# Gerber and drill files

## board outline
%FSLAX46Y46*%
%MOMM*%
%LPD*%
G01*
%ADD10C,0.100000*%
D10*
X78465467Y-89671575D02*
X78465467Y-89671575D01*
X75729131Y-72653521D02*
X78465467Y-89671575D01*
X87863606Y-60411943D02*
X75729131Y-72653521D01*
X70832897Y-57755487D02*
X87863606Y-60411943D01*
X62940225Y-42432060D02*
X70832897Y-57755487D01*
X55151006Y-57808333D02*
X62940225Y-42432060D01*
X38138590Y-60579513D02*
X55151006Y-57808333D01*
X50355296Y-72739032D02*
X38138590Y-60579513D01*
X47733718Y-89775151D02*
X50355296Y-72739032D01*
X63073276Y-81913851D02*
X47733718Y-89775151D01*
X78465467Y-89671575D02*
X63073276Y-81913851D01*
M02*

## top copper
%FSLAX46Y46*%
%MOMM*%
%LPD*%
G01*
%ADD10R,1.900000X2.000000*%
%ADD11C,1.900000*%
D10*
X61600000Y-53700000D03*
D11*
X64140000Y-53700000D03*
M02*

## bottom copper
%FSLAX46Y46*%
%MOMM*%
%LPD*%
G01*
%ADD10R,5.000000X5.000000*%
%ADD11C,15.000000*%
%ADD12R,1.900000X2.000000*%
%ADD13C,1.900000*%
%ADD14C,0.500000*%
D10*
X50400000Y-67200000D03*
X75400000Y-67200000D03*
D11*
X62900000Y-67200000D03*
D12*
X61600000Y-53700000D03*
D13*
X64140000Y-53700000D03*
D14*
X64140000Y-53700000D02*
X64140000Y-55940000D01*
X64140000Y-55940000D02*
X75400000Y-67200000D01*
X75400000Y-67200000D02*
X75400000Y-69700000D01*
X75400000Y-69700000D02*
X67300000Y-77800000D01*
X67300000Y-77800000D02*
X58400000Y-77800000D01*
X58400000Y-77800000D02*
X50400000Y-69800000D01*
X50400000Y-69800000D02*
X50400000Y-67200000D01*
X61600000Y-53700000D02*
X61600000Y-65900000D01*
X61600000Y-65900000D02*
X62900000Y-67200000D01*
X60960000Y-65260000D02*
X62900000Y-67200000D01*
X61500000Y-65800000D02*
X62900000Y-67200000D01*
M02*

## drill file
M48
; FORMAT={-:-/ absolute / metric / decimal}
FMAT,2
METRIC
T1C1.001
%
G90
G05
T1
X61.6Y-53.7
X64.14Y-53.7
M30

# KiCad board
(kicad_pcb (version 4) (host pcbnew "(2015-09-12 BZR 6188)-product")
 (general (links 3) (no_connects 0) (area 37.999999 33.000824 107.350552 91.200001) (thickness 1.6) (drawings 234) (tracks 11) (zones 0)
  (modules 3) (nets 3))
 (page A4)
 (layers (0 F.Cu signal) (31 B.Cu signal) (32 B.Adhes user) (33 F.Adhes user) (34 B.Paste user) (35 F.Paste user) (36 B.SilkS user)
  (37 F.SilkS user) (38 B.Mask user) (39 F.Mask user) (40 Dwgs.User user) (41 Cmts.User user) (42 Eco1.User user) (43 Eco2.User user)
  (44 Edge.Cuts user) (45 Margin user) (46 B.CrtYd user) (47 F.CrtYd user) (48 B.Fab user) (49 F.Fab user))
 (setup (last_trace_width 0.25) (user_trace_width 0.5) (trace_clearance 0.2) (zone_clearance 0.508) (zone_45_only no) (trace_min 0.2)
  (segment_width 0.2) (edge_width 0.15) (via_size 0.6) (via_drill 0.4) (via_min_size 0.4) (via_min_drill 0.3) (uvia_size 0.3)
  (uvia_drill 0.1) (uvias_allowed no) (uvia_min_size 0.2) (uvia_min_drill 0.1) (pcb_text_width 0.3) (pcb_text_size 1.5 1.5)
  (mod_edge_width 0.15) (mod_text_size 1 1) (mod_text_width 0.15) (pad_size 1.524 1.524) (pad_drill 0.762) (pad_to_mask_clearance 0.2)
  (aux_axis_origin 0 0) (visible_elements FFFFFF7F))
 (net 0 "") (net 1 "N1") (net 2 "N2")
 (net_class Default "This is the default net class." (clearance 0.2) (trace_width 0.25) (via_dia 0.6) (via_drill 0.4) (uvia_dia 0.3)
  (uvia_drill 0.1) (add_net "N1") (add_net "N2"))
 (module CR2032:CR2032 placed (layer B.Cu) (at 62.9 67.2)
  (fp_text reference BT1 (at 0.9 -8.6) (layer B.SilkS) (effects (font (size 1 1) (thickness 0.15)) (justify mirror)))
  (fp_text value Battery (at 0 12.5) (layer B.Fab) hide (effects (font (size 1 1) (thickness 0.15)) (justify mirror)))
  (pad 1 smd rect (at -12.5 0) (size 5 5) (layers B.Cu B.Paste B.Mask) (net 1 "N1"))
  (pad 1 smd rect (at 12.5 0) (size 5 5) (layers B.Cu B.Paste B.Mask) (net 1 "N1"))
  (pad 2 smd circle (at 0 0) (size 15 15) (layers B.Cu B.Paste B.Mask) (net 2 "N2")))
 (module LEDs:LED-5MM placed (layer F.Cu) (at 61.6 53.7)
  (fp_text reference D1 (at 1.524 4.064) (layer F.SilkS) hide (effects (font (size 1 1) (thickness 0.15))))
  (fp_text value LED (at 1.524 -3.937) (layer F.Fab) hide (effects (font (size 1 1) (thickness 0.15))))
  (pad 1 thru_hole rect (at 0 0 90) (size 2 1.9) (drill 1.00076) (layers *.Cu *.Mask F.SilkS) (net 2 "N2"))
  (pad 2 thru_hole circle (at 2.54 0) (size 1.9 1.9) (drill 1.00076) (layers *.Cu *.Mask F.SilkS) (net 1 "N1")))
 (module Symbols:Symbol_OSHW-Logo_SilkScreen (layer B.Cu) (at 71.9 78.5 180)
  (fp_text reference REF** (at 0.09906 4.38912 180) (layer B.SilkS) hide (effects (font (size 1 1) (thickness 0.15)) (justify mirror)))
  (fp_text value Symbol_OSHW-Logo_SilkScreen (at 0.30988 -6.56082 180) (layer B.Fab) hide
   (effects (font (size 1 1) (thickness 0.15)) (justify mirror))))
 (gr_line (start 78.465467 89.671575) (end 78.465467 89.671575) (layer Edge.Cuts) (width 0.1))
 (gr_line (start 75.729131 72.653521) (end 78.465467 89.671575) (layer Edge.Cuts) (width 0.1))
 (gr_line (start 87.863606 60.411943) (end 75.729131 72.653521) (layer Edge.Cuts) (width 0.1))
 (gr_line (start 70.832897 57.755487) (end 87.863606 60.411943) (layer Edge.Cuts) (width 0.1))
 (gr_line (start 62.940225 42.43206) (end 70.832897 57.755487) (layer Edge.Cuts) (width 0.1))
 (gr_line (start 55.151006 57.808333) (end 62.940225 42.43206) (layer Edge.Cuts) (width 0.1))
 (gr_line (start 38.13859 60.579513) (end 55.151006 57.808333) (layer Edge.Cuts) (width 0.1))
 (gr_line (start 50.355296 72.739032) (end 38.13859 60.579513) (layer Edge.Cuts) (width 0.1))
 (gr_line (start 47.733718 89.775151) (end 50.355296 72.739032) (layer Edge.Cuts) (width 0.1))
 (gr_line (start 63.073276 81.913851) (end 47.733718 89.775151) (layer Edge.Cuts) (width 0.1))
 (gr_line (start 78.465467 89.671575) (end 63.073276 81.913851) (layer Edge.Cuts) (width 0.1))
 (segment (start 64.14 53.7) (end 64.14 55.94) (width 0.5) (layer B.Cu) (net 1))
 (segment (start 64.14 55.94) (end 75.4 67.2) (width 0.5) (layer B.Cu) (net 1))
 (segment (start 75.4 67.2) (end 75.4 69.7) (width 0.5) (layer B.Cu) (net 1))
 (segment (start 75.4 69.7) (end 67.3 77.8) (width 0.5) (layer B.Cu) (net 1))
 (segment (start 67.3 77.8) (end 58.4 77.8) (width 0.5) (layer B.Cu) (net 1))
 (segment (start 58.4 77.8) (end 50.4 69.8) (width 0.5) (layer B.Cu) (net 1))
 (segment (start 50.4 69.8) (end 50.4 67.2) (width 0.5) (layer B.Cu) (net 1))
 (segment (start 61.6 53.7) (end 61.6 65.9) (width 0.5) (layer B.Cu) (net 2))
 (segment (start 61.6 65.9) (end 62.9 67.2) (width 0.5) (layer B.Cu) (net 2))
 (segment (start 60.96 65.26) (end 62.9 67.2) (width 0.5) (layer B.Cu) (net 2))
 (segment (start 61.5 65.8) (end 62.9 67.2) (width 0.5) (layer B.Cu) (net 2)))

